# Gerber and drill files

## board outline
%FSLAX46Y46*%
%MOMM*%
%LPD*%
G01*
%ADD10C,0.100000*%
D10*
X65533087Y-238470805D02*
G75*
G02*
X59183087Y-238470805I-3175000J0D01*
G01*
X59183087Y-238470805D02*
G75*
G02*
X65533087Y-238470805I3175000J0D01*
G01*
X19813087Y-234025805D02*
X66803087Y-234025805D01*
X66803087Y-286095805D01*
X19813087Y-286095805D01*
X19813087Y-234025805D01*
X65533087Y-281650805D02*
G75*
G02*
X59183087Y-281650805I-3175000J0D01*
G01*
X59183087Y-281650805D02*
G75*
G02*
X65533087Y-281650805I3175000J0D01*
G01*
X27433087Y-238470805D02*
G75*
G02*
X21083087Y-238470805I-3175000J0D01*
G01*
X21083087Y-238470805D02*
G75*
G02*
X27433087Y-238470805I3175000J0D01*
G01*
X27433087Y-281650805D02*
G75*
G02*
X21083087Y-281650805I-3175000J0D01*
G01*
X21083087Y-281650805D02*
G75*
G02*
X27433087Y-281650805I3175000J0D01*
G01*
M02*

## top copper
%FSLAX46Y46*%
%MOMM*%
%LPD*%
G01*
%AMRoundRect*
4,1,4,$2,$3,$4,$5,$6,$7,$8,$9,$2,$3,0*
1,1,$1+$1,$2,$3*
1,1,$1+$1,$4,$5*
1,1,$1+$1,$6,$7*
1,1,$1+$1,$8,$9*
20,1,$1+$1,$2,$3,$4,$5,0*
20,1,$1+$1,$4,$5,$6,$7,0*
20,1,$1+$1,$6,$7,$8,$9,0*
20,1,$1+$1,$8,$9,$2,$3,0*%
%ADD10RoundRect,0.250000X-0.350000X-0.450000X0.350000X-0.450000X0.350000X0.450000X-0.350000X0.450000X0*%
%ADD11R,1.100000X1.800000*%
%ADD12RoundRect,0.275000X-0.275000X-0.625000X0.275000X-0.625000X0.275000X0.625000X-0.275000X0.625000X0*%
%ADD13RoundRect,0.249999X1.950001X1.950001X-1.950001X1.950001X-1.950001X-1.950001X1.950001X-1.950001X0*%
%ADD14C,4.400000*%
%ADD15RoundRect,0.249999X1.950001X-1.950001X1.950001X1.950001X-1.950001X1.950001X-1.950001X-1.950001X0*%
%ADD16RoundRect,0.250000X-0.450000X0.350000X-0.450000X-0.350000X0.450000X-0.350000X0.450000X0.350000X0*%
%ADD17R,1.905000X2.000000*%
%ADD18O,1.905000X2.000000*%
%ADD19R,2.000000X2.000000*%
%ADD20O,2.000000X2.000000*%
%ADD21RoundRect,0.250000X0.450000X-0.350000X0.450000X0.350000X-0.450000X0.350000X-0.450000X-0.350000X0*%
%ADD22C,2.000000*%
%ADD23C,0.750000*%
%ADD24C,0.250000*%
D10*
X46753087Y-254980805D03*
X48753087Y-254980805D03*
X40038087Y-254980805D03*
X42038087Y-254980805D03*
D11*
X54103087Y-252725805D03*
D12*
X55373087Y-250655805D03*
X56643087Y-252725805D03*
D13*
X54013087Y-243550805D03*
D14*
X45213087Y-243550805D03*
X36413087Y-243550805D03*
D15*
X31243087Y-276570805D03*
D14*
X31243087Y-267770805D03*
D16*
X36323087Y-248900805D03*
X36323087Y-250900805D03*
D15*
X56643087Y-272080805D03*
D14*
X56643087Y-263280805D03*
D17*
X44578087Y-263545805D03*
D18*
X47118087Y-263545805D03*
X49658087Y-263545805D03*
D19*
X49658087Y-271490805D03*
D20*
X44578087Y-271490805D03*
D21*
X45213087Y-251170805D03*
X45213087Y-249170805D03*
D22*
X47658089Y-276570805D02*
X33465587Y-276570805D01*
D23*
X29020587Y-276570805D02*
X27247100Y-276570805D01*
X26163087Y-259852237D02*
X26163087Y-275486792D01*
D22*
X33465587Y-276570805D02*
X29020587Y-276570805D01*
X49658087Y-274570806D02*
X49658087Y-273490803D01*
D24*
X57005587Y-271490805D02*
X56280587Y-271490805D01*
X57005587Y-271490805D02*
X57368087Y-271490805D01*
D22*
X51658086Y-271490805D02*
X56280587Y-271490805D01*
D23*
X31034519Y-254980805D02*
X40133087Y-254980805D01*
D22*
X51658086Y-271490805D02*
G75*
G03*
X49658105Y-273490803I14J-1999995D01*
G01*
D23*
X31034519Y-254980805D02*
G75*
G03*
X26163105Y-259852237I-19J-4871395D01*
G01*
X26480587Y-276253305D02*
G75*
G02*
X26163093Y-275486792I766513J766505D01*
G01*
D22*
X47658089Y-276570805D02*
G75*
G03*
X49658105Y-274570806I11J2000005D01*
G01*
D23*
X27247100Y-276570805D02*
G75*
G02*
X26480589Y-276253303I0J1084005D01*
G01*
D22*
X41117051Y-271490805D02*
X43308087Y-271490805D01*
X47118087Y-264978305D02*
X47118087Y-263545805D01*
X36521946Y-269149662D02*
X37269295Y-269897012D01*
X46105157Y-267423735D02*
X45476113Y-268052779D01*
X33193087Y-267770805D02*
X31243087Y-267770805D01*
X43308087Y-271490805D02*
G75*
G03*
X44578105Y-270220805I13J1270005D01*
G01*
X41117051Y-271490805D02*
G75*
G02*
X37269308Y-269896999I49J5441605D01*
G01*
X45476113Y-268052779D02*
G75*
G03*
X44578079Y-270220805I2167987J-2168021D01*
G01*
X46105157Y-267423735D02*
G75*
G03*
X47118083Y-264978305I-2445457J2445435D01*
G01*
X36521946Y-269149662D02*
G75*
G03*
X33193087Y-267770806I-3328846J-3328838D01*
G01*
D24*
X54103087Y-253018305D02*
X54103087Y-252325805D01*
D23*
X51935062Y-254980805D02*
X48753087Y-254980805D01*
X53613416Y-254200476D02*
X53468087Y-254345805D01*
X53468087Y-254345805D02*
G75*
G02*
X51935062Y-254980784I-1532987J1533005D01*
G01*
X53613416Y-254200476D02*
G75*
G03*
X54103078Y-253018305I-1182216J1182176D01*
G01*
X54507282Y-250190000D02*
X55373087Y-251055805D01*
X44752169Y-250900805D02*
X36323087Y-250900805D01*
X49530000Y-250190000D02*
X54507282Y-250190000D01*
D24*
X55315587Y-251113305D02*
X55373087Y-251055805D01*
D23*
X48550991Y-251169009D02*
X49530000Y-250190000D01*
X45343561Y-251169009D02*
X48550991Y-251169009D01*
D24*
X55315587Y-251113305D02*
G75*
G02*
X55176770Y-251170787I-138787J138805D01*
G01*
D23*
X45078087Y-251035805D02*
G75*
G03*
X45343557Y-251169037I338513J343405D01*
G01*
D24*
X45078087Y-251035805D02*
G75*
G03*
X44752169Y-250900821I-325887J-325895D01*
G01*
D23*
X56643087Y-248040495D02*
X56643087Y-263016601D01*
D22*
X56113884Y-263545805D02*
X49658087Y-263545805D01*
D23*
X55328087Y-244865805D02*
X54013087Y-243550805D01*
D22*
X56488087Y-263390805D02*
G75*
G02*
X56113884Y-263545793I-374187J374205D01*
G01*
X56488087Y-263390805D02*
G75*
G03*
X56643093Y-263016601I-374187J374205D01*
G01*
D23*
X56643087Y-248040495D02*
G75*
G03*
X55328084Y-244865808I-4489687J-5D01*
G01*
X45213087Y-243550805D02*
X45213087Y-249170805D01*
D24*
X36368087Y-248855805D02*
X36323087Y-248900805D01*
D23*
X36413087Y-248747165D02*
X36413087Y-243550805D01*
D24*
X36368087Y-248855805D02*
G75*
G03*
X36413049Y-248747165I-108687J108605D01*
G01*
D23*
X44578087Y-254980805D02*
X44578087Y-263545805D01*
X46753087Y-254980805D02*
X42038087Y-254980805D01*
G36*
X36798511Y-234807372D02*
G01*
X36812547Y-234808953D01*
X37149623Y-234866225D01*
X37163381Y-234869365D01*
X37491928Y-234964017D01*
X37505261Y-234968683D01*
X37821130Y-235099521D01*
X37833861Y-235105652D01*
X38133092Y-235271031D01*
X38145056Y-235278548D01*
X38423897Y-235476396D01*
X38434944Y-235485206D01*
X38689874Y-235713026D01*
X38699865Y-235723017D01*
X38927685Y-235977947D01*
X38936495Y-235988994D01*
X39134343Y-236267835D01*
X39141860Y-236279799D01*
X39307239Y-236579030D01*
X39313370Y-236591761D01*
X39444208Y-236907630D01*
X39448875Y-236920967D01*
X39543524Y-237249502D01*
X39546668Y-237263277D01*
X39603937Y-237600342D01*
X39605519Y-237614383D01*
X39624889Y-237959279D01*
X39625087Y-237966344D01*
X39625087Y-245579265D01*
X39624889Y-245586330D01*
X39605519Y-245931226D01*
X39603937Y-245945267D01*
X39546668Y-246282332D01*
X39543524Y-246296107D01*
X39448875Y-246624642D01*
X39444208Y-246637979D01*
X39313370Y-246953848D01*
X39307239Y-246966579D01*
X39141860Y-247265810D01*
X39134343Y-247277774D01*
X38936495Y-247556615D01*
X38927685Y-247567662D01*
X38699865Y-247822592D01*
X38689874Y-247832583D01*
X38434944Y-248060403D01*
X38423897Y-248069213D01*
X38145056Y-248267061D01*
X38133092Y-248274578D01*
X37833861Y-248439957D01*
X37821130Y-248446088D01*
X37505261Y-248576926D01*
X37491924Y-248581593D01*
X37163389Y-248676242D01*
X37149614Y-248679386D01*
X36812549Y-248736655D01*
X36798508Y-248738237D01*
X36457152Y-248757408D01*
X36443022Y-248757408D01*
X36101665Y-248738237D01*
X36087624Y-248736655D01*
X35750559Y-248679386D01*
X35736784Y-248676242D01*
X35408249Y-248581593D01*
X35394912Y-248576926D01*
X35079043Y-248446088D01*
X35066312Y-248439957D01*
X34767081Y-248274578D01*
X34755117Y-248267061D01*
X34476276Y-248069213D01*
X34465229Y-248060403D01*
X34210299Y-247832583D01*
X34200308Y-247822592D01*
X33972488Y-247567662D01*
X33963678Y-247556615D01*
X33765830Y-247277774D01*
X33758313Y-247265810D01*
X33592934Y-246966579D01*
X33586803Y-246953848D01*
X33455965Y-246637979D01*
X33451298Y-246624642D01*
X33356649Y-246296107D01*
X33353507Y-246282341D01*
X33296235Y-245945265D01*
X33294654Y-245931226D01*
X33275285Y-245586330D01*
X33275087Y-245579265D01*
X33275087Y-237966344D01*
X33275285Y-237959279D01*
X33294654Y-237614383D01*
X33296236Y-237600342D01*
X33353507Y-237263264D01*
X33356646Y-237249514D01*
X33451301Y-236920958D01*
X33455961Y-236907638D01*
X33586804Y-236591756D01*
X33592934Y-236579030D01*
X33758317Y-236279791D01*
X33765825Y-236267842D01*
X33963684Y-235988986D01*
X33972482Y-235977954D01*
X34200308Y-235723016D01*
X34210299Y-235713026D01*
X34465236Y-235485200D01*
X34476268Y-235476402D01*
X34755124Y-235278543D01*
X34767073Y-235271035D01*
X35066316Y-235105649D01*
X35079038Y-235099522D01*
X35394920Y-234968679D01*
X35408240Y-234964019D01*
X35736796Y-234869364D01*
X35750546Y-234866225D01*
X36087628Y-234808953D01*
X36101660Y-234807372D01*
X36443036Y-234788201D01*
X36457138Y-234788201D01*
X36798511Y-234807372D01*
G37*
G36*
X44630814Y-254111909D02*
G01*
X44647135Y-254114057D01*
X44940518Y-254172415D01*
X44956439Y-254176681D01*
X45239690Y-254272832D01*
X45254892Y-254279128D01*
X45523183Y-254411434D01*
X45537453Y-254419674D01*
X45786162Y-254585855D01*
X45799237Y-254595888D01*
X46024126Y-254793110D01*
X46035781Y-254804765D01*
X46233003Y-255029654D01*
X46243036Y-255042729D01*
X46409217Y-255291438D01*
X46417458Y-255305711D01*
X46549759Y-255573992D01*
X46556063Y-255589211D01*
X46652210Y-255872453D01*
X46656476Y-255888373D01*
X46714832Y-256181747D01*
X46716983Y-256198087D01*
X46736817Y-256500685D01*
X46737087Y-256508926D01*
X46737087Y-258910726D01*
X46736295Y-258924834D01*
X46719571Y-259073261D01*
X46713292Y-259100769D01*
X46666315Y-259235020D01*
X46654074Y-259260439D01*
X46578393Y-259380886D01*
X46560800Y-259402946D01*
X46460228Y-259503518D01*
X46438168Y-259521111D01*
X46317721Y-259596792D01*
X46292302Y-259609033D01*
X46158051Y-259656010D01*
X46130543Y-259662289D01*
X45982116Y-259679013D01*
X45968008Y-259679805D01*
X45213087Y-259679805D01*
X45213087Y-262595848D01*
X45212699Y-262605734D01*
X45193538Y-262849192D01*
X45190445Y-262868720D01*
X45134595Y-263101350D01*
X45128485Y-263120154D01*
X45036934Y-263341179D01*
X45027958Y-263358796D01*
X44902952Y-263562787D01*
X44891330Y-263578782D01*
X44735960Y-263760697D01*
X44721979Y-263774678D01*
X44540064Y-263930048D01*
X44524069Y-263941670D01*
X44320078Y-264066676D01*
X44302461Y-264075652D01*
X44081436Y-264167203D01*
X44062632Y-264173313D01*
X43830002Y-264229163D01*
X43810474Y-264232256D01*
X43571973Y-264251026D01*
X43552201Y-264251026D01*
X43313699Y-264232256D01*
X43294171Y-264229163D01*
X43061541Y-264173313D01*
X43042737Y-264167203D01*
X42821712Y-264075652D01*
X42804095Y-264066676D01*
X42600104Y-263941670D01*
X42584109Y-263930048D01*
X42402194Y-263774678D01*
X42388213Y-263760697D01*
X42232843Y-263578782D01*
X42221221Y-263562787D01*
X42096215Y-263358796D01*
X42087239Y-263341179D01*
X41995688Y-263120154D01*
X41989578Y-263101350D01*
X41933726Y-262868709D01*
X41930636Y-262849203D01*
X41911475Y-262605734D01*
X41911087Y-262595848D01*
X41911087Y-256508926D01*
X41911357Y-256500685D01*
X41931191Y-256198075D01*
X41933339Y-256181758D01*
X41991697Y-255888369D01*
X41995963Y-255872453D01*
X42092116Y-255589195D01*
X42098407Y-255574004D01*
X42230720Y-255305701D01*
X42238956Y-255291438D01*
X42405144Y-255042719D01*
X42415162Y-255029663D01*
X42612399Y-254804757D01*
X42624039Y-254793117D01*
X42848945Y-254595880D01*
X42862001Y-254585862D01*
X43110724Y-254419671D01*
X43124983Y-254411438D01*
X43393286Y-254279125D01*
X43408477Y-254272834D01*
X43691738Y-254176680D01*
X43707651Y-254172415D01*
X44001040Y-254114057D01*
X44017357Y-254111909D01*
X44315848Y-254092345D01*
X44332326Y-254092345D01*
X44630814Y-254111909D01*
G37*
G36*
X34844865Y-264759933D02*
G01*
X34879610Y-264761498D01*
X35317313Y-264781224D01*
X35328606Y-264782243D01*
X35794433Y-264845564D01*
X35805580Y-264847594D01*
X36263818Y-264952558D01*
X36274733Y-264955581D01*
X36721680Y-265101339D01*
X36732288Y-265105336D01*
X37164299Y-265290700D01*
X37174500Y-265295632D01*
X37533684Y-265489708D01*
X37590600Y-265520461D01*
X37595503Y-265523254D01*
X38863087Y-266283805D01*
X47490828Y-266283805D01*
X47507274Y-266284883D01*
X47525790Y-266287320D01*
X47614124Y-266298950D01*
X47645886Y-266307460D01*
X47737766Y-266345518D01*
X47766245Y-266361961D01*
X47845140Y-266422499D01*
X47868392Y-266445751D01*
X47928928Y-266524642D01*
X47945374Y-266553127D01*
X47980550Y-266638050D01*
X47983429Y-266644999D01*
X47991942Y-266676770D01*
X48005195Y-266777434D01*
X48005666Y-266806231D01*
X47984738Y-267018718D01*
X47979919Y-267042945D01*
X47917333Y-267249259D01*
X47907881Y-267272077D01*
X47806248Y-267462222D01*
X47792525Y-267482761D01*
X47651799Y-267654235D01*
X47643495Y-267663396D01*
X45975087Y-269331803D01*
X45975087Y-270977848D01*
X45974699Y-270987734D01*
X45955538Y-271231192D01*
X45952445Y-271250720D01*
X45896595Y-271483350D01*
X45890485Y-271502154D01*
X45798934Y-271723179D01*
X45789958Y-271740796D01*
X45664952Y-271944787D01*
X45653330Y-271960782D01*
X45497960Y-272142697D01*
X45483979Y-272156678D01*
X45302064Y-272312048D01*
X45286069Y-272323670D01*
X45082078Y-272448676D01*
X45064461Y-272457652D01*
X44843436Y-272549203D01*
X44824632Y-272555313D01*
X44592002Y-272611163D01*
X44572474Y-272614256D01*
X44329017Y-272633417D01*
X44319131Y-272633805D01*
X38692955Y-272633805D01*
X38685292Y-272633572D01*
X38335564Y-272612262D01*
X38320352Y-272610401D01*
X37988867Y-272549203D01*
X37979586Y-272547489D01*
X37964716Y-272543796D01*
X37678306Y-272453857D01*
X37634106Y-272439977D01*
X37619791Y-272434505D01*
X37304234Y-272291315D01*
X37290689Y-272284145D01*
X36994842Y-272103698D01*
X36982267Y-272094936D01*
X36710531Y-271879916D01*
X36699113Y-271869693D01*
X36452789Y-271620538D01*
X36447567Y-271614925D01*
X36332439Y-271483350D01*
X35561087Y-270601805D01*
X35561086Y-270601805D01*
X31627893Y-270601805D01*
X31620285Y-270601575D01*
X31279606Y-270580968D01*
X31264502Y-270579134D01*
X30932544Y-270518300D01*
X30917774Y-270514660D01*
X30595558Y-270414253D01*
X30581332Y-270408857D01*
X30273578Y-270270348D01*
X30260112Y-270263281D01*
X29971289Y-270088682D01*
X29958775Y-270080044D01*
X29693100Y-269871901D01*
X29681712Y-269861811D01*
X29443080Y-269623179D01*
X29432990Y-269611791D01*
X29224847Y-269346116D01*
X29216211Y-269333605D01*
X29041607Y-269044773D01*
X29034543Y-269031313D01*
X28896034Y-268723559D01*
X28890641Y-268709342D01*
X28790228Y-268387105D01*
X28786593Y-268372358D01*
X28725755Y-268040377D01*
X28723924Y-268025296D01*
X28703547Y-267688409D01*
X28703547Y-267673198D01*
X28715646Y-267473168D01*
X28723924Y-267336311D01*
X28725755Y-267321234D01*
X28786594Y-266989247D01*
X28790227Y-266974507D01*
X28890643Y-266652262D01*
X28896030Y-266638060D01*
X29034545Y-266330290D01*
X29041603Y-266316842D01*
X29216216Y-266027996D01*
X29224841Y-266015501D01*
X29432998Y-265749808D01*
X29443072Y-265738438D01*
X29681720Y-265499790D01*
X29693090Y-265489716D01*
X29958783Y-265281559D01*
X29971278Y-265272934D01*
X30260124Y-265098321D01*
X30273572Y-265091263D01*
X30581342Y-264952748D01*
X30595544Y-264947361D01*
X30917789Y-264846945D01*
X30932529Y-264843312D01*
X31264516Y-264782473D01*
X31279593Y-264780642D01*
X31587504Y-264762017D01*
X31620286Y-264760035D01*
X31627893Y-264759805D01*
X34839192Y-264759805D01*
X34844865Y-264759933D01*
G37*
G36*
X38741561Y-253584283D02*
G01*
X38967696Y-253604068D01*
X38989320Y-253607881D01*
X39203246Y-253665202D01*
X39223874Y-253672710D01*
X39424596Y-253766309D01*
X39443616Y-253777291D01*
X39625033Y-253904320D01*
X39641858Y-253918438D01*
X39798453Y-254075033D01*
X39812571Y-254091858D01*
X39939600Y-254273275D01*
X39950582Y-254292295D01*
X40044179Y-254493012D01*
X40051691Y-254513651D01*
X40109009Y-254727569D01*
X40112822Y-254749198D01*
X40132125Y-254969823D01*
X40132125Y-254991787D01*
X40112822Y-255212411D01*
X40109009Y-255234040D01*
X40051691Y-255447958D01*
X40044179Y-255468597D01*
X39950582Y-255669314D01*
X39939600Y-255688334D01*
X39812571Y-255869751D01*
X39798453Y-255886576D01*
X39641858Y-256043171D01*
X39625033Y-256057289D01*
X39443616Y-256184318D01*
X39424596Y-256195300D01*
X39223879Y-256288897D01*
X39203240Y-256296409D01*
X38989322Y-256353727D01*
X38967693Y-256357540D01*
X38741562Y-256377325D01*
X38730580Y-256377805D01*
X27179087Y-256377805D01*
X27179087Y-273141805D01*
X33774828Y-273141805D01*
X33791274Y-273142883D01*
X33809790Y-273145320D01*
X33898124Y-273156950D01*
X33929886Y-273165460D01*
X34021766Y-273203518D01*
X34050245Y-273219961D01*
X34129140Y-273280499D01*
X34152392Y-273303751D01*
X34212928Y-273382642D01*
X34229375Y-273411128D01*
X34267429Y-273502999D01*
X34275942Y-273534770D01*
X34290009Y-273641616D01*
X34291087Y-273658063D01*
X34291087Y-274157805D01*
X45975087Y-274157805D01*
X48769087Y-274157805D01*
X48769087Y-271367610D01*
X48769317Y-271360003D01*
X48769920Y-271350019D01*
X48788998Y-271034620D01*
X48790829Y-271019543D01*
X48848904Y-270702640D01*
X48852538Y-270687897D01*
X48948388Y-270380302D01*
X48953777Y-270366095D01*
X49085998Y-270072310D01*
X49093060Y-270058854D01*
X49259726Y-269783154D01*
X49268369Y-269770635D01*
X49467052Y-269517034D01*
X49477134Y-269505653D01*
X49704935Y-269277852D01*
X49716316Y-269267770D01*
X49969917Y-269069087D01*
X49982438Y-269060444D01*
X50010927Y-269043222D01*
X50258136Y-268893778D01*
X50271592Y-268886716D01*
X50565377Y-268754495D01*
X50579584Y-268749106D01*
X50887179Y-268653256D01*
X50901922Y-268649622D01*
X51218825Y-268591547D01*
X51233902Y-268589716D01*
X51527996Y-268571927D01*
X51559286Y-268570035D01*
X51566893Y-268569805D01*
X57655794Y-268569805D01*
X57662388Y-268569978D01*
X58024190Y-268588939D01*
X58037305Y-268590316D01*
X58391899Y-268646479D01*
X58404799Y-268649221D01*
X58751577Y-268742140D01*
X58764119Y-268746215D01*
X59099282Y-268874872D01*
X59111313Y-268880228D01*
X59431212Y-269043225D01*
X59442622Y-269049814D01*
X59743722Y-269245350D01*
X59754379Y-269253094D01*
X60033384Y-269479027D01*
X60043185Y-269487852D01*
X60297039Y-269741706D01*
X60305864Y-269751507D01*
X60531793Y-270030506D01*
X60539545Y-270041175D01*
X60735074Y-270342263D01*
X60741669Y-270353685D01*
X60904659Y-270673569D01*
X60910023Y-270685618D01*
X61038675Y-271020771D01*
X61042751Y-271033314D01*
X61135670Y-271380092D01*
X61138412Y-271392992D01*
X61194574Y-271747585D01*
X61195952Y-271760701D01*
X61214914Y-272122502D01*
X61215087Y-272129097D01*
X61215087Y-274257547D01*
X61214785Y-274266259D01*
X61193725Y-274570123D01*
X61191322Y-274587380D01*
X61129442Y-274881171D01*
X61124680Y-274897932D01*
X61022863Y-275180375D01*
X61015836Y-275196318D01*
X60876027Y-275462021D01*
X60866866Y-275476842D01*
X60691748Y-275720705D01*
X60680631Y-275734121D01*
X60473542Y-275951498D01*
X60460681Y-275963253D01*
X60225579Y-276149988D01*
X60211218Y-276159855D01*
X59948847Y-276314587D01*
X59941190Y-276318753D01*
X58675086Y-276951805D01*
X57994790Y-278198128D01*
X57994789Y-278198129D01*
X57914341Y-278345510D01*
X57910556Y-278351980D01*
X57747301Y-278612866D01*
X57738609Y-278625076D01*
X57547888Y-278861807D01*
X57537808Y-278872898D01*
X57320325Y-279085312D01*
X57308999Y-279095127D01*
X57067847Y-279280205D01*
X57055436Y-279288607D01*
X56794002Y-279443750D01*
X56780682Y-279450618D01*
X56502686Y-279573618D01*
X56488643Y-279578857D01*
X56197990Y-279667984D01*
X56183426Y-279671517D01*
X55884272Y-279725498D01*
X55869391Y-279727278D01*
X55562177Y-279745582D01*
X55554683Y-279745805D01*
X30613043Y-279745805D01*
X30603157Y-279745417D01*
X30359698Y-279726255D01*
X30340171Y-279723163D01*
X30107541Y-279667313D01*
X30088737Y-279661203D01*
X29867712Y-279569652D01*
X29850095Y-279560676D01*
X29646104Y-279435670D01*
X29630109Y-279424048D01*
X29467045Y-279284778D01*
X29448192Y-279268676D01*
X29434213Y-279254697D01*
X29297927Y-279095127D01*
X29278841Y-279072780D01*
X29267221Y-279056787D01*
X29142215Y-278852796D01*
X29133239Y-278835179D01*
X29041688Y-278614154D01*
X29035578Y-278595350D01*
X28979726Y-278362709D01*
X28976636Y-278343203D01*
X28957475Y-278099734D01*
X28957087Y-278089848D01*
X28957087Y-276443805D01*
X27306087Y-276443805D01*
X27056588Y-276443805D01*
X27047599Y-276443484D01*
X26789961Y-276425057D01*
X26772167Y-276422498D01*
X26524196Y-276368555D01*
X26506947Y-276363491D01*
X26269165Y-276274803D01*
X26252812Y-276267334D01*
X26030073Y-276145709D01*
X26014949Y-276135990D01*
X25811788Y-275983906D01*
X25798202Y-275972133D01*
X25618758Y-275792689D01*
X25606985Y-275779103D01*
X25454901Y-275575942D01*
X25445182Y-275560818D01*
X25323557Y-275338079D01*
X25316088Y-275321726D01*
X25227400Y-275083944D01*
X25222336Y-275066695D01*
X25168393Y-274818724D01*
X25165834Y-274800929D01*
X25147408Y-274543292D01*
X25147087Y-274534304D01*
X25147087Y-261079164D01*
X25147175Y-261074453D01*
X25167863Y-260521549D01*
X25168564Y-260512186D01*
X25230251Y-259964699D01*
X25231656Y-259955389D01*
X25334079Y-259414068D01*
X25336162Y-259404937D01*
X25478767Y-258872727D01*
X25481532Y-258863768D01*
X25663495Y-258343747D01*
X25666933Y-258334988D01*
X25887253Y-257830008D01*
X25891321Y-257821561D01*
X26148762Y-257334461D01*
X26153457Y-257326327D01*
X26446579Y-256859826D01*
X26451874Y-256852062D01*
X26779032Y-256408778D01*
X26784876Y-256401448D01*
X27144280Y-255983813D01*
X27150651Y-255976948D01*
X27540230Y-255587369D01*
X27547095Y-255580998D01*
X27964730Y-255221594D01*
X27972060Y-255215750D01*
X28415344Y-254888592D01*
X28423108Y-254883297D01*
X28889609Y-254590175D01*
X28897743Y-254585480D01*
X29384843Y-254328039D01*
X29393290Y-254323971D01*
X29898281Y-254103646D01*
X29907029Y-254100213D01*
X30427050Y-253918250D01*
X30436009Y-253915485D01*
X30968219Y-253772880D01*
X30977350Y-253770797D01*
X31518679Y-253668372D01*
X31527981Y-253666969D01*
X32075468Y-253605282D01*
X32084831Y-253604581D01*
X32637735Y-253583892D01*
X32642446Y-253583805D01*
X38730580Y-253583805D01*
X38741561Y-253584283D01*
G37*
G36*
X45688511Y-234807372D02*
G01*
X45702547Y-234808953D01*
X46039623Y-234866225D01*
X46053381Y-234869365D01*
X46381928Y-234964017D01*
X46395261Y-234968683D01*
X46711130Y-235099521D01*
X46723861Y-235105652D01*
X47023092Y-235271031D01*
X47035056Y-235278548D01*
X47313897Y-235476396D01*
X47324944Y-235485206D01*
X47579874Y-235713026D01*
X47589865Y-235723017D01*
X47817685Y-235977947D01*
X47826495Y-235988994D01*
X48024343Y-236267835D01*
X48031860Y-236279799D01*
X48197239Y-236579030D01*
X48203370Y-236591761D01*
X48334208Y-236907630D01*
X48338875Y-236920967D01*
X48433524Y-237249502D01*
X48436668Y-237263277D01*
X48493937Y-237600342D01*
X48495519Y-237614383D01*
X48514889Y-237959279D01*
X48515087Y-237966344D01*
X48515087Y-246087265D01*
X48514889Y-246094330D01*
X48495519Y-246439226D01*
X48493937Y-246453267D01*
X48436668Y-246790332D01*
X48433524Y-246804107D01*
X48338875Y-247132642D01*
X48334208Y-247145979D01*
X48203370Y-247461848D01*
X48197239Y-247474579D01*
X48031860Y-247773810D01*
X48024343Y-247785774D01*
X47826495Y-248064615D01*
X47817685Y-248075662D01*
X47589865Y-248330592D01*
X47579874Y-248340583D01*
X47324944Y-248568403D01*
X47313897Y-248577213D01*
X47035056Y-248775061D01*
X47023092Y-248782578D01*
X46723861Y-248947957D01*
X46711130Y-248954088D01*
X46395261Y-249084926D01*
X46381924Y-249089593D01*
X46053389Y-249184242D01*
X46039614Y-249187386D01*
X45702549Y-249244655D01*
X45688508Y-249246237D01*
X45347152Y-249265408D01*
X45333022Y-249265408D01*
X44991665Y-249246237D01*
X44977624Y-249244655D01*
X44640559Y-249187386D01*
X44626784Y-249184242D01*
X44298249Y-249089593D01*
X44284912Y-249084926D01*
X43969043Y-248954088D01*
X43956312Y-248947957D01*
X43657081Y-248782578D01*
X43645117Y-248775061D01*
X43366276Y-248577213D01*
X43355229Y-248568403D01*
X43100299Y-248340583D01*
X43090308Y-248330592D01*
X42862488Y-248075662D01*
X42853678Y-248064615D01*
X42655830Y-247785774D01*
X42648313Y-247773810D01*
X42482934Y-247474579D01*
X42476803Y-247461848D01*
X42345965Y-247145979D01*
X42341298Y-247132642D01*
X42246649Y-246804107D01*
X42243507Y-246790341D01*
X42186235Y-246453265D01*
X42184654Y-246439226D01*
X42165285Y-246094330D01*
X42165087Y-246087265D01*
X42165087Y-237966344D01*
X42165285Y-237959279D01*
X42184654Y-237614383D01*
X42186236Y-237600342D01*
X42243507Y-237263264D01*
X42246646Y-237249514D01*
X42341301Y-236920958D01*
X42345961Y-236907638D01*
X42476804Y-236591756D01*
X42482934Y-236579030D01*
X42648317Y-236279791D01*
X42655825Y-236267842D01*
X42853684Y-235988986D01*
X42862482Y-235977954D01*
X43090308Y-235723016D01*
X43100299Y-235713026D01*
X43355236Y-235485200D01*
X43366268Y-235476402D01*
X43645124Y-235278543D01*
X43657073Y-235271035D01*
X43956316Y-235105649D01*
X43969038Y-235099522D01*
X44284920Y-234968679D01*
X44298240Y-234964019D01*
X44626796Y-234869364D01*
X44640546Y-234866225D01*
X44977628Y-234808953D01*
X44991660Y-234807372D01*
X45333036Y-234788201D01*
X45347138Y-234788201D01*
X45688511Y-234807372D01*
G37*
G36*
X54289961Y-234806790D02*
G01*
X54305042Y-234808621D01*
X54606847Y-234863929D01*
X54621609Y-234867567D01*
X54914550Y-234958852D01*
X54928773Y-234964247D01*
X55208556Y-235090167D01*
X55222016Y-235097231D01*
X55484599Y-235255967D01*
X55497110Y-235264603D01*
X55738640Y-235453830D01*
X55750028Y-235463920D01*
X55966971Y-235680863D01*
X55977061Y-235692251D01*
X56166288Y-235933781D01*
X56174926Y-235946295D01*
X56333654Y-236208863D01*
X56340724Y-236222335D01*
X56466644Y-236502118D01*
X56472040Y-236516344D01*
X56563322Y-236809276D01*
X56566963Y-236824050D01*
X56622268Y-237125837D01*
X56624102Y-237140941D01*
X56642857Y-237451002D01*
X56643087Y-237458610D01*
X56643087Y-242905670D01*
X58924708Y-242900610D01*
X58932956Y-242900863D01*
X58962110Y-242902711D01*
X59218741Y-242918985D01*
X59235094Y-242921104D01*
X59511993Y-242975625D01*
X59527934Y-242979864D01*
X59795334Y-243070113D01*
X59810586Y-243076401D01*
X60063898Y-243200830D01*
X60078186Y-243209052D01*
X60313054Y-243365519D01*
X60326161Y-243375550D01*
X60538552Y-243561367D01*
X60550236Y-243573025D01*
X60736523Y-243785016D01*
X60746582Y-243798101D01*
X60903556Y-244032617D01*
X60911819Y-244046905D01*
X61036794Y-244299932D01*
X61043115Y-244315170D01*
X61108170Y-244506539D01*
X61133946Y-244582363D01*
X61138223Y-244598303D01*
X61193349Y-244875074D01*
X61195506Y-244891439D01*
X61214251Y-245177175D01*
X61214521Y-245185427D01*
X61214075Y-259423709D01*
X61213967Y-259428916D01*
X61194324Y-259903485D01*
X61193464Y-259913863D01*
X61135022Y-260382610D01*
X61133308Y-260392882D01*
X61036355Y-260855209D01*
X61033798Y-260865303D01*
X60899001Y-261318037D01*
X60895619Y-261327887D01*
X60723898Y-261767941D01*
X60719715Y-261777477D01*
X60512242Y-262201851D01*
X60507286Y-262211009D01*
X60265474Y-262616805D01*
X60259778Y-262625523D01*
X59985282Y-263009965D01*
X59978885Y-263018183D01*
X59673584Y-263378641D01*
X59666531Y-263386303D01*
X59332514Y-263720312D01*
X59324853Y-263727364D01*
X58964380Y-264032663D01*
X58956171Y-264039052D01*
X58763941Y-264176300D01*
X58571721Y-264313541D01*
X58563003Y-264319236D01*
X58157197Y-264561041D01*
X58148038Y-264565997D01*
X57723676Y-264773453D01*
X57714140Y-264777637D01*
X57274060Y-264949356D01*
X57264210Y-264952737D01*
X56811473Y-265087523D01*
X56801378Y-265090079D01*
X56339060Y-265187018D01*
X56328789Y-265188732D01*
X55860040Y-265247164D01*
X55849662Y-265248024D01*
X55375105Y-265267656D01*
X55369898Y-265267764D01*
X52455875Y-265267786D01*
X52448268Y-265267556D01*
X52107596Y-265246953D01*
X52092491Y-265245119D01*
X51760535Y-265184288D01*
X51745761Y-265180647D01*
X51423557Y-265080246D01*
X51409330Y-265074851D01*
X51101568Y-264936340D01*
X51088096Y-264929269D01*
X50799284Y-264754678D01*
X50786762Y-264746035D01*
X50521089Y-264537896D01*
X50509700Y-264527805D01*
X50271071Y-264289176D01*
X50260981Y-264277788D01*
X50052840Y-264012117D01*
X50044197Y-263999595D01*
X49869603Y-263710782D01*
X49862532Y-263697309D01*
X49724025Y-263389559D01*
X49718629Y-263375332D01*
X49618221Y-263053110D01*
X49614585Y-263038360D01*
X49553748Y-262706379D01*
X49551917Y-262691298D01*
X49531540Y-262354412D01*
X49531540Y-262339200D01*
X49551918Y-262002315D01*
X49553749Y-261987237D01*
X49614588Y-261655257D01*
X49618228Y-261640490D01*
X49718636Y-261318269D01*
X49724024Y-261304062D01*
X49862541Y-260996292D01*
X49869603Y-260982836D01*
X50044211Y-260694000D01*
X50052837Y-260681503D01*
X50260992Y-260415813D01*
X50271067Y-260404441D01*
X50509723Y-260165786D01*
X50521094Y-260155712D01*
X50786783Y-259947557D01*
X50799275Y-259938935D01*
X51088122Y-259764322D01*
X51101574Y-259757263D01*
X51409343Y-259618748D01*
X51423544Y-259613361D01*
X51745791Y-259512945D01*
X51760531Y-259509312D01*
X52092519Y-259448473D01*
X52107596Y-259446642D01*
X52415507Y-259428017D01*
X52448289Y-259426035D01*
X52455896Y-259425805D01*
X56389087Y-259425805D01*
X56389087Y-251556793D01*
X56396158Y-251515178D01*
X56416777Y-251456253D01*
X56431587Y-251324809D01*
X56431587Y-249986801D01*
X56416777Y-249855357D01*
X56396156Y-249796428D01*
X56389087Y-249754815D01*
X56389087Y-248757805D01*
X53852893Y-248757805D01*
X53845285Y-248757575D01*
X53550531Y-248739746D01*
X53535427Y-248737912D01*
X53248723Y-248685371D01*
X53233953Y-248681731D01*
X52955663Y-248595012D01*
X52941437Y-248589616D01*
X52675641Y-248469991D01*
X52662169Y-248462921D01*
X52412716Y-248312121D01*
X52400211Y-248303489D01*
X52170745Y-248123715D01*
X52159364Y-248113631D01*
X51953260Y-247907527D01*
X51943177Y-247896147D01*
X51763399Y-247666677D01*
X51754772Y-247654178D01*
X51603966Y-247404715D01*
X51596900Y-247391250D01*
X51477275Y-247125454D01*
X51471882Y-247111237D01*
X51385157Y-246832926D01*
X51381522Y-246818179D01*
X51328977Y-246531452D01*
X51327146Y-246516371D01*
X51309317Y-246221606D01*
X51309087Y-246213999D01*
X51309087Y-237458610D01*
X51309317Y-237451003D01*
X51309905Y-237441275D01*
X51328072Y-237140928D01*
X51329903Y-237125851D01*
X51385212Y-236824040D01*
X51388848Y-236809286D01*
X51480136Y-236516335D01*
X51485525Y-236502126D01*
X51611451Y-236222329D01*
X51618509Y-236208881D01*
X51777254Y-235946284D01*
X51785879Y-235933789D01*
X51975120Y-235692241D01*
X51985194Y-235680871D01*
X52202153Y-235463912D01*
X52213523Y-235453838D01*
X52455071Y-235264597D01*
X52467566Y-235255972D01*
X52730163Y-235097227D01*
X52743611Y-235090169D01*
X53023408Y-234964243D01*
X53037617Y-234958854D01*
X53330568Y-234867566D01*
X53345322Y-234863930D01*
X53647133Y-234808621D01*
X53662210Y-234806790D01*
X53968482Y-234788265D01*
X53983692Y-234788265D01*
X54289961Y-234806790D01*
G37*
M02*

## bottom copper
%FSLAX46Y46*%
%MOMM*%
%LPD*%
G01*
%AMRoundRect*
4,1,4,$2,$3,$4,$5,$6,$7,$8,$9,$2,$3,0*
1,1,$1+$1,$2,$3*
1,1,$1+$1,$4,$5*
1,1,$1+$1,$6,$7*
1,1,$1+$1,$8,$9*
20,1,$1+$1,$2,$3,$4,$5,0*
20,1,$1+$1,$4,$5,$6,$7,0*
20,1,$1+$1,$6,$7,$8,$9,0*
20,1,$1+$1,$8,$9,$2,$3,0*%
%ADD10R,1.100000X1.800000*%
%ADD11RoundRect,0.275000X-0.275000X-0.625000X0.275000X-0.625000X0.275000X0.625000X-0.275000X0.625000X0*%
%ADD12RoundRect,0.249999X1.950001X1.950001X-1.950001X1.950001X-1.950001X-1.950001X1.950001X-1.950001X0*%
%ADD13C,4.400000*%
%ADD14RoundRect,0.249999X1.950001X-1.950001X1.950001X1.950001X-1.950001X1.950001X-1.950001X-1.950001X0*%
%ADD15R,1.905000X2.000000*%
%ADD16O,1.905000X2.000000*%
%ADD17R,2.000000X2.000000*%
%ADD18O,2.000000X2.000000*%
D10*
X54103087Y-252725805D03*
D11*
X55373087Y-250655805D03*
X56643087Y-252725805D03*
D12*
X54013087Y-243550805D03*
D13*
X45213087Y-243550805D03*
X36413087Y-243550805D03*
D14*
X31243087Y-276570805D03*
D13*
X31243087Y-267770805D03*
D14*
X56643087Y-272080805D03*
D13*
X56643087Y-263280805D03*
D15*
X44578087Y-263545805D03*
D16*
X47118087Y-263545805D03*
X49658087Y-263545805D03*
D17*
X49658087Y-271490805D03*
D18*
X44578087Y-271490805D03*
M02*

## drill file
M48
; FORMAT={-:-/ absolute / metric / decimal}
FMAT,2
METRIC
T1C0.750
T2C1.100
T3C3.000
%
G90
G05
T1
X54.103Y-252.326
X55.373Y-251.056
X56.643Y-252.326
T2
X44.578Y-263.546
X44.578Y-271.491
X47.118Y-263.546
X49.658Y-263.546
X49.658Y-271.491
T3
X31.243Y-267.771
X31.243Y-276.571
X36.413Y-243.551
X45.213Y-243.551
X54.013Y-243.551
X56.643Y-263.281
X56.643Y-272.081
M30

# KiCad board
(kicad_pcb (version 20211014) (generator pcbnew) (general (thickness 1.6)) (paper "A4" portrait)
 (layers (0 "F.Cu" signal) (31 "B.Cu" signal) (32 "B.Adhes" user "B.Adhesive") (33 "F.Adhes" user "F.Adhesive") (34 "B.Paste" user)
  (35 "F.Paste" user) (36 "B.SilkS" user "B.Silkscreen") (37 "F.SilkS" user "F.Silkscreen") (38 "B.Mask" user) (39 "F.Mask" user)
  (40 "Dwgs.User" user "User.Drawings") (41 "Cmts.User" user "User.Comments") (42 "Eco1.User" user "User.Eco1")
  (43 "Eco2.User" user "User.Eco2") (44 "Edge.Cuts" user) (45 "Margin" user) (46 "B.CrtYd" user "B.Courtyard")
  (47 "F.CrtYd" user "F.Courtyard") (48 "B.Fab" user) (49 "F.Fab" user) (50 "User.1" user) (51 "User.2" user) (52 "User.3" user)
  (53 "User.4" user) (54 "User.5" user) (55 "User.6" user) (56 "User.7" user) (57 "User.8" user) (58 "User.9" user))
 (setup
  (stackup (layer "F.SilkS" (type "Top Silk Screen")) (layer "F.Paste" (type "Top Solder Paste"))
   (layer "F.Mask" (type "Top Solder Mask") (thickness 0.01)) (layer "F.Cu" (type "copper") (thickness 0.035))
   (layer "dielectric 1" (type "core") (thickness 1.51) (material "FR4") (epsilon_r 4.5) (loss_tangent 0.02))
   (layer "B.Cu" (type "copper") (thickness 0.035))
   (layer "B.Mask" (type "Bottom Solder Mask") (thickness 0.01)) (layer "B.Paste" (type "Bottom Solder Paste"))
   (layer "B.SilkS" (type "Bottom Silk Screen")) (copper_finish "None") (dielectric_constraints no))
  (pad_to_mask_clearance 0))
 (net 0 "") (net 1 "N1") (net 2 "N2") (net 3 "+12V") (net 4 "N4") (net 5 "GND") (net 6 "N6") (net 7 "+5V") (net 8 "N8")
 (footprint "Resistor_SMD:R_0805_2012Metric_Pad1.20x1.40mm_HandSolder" (layer "F.Cu") (at 47.753087 254.980805)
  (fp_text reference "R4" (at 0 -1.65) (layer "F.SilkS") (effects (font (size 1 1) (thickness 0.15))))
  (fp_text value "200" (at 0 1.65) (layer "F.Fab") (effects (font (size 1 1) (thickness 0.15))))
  (pad "1" smd roundrect (at -1 0) (size 1.2 1.4) (layers "F.Cu" "F.Paste" "F.Mask") (roundrect_rratio 0.2083333333) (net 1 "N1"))
  (pad "2" smd roundrect (at 1 0) (size 1.2 1.4) (layers "F.Cu" "F.Paste" "F.Mask") (roundrect_rratio 0.2083333333) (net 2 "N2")))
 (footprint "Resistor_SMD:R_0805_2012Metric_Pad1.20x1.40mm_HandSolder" (layer "F.Cu") (at 41.038087 254.980805)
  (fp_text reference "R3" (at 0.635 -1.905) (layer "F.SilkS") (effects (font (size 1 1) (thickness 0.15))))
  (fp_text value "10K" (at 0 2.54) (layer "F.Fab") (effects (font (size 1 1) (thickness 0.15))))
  (pad "1" smd roundrect (at -1 0) (size 1.2 1.4) (layers "F.Cu" "F.Paste" "F.Mask") (roundrect_rratio 0.2083333333) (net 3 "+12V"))
  (pad "2" smd roundrect (at 1 0) (size 1.2 1.4) (layers "F.Cu" "F.Paste" "F.Mask") (roundrect_rratio 0.2083333333) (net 1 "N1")))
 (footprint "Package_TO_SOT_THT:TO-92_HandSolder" (layer "F.Cu") (at 54.103087 252.325805)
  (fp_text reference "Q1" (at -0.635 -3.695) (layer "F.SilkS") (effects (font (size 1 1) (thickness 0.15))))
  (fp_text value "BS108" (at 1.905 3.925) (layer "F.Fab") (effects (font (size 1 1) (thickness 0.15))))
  (pad "1" thru_hole rect (at 0 0) (size 1.1 1.8) (drill 0.75 (offset 0 0.4)) (layers *.Cu *.Mask) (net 2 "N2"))
  (pad "2" thru_hole roundrect (at 1.27 -1.27) (size 1.1 1.8) (drill 0.75 (offset 0 -0.4)) (layers *.Cu *.Mask) (roundrect_rratio 0.25)
   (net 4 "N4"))
  (pad "3" thru_hole roundrect (at 2.54 0) (size 1.1 1.8) (drill 0.75 (offset 0 0.4)) (layers *.Cu *.Mask) (roundrect_rratio 0.25)
   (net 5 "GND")))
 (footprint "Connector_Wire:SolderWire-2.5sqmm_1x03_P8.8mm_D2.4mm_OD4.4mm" (layer "F.Cu") (at 54.013087 243.550805 180)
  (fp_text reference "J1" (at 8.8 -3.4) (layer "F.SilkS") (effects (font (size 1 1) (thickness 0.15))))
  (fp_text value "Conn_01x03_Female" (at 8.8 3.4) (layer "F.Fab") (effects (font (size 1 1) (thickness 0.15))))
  (pad "1" thru_hole roundrect (at 0 0 180) (size 4.4 4.4) (drill 3) (layers *.Cu *.Mask) (roundrect_rratio 0.05681795455) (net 5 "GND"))
  (pad "2" thru_hole circle (at 8.8 0 180) (size 4.4 4.4) (drill 3) (layers *.Cu *.Mask) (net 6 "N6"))
  (pad "3" thru_hole circle (at 17.6 0 180) (size 4.4 4.4) (drill 3) (layers *.Cu *.Mask) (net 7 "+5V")))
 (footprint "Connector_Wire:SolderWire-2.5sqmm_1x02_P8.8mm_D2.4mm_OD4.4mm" (layer "F.Cu") (at 31.243087 276.570805 90)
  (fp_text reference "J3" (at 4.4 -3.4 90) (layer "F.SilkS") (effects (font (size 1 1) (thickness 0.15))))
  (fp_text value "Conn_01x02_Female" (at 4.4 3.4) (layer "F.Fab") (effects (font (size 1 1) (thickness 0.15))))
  (pad "1" thru_hole roundrect (at 0 0 90) (size 4.4 4.4) (drill 3) (layers *.Cu *.Mask) (roundrect_rratio 0.05681795455) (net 3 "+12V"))
  (pad "2" thru_hole circle (at 8.8 0 90) (size 4.4 4.4) (drill 3) (layers *.Cu *.Mask) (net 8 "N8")))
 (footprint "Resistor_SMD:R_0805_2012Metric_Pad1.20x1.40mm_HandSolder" (layer "F.Cu") (at 36.323087 249.900805 -90)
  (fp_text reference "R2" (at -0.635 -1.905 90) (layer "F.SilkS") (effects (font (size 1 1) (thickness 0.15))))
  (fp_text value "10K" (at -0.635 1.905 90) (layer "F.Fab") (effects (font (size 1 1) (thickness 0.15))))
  (pad "1" smd roundrect (at -1 0 270) (size 1.2 1.4) (layers "F.Cu" "F.Paste" "F.Mask") (roundrect_rratio 0.2083333333) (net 7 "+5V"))
  (pad "2" smd roundrect (at 1 0 270) (size 1.2 1.4) (layers "F.Cu" "F.Paste" "F.Mask") (roundrect_rratio 0.2083333333) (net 4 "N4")))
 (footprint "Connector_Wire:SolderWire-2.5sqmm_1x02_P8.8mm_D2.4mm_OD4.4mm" (layer "F.Cu") (at 56.643087 272.080805 90)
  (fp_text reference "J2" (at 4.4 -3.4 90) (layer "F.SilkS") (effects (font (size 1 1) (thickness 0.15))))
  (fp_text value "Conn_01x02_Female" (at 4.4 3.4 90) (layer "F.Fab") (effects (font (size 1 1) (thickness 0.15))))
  (pad "1" thru_hole roundrect (at 0 0 90) (size 4.4 4.4) (drill 3) (layers *.Cu *.Mask) (roundrect_rratio 0.05681795455) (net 3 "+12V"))
  (pad "2" thru_hole circle (at 8.8 0 90) (size 4.4 4.4) (drill 3) (layers *.Cu *.Mask) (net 5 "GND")))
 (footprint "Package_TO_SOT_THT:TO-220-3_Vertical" (layer "F.Cu") (at 44.578087 263.545805)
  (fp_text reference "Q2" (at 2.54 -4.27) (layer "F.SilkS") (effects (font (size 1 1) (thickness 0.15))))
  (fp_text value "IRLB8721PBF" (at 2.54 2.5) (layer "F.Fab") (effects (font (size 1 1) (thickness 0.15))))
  (pad "1" thru_hole rect (at 0 0) (size 1.905 2) (drill 1.1) (layers *.Cu *.Mask) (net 1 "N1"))
  (pad "2" thru_hole oval (at 2.54 0) (size 1.905 2) (drill 1.1) (layers *.Cu *.Mask) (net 8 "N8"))
  (pad "3" thru_hole oval (at 5.08 0) (size 1.905 2) (drill 1.1) (layers *.Cu *.Mask) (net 5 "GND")))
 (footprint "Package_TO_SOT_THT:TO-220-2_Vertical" (layer "F.Cu") (at 49.658087 271.490805 180)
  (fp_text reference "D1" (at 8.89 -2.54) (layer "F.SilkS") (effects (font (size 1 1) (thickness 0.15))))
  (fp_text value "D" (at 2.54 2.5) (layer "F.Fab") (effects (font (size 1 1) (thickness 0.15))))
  (pad "1" thru_hole rect (at 0 0 180) (size 2 2) (drill 1.1) (layers *.Cu *.Mask) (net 3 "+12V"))
  (pad "2" thru_hole oval (at 5.08 0 180) (size 2 2) (drill 1.1) (layers *.Cu *.Mask) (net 8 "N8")))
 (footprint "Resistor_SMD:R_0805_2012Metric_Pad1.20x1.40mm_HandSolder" (layer "F.Cu") (at 45.213087 250.170805 90)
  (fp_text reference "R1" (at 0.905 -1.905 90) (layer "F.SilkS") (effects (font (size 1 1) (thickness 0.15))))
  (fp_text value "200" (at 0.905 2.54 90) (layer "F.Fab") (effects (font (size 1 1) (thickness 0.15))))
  (pad "1" smd roundrect (at -1 0 90) (size 1.2 1.4) (layers "F.Cu" "F.Paste" "F.Mask") (roundrect_rratio 0.2083333333) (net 4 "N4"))
  (pad "2" smd roundrect (at 1 0 90) (size 1.2 1.4) (layers "F.Cu" "F.Paste" "F.Mask") (roundrect_rratio 0.2083333333) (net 6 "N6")))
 (gr_circle (center 62.358087 238.470805) (end 64.898087 240.375805) (layer "Edge.Cuts") (width 0.1) (fill none))
 (gr_rect (start 19.813087 234.025805) (end 66.803087 286.095805) (layer "Edge.Cuts") (width 0.1) (fill none))
 (gr_circle (center 62.358087 281.650805) (end 64.898087 283.555805) (layer "Edge.Cuts") (width 0.1) (fill none))
 (gr_circle (center 24.258087 238.470805) (end 26.798087 240.375805) (layer "Edge.Cuts") (width 0.1) (fill none))
 (gr_circle (center 24.258087 281.650805) (end 26.798087 283.555805) (layer "Edge.Cuts") (width 0.1) (fill none))
 (segment (start 47.658089 276.570805) (end 33.465587 276.570805) (width 2) (layer "F.Cu") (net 3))
 (segment (start 29.020587 276.570805) (end 27.2471 276.570805) (width 0.75) (layer "F.Cu") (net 3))
 (segment (start 26.163087 259.852237) (end 26.163087 275.486792) (width 0.75) (layer "F.Cu") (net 3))
 (segment (start 33.465587 276.570805) (end 29.020587 276.570805) (width 2) (layer "F.Cu") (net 3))
 (segment (start 49.658087 274.570806) (end 49.658087 273.490803) (width 2) (layer "F.Cu") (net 3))
 (segment (start 57.005587 271.490805) (end 56.280587 271.490805) (width 0.25) (layer "F.Cu") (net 3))
 (segment (start 57.005587 271.490805) (end 57.368087 271.490805) (width 0.25) (layer "F.Cu") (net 3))
 (segment (start 51.658086 271.490805) (end 56.280587 271.490805) (width 2) (layer "F.Cu") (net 3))
 (segment (start 31.034519 254.980805) (end 40.133087 254.980805) (width 0.75) (layer "F.Cu") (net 3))
 (arc (start 51.658086 271.490805) (mid 50.243874 272.07659) (end 49.658087 273.490803) (width 2) (layer "F.Cu") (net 3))
 (arc (start 31.034519 254.980805) (mid 27.589896 256.407614) (end 26.163087 259.852237) (width 0.75) (layer "F.Cu") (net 3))
 (arc (start 26.480587 276.253305) (mid 26.245603 275.901625) (end 26.163087 275.486792) (width 0.75) (layer "F.Cu") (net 3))
 (arc (start 47.658089 276.570805) (mid 49.072302 275.985018) (end 49.658087 274.570806) (width 2) (layer "F.Cu") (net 3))
 (arc (start 27.2471 276.570805) (mid 26.832267 276.488289) (end 26.480587 276.253305) (width 0.75) (layer "F.Cu") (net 3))
 (segment (start 41.117051 271.490805) (end 43.308087 271.490805) (width 2) (layer "F.Cu") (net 8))
 (segment (start 47.118087 264.978305) (end 47.118087 263.545805) (width 2) (layer "F.Cu") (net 8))
 (segment (start 36.521946 269.149662) (end 37.269295 269.897012) (width 2) (layer "F.Cu") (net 8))
 (segment (start 46.105157 267.423735) (end 45.476113 268.052779) (width 2) (layer "F.Cu") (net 8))
 (segment (start 33.193087 267.770805) (end 31.243087 267.770805) (width 2) (layer "F.Cu") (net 8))
 (arc (start 43.308087 271.490805) (mid 44.206113 271.11883) (end 44.578087 270.220805) (width 2) (layer "F.Cu") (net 8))
 (arc (start 41.117051 271.490805) (mid 39.034661 271.076591) (end 37.269295 269.897012) (width 2) (layer "F.Cu") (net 8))
 (arc (start 45.476113 268.052779) (mid 44.811477 269.047477) (end 44.578087 270.220805) (width 2) (layer "F.Cu") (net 8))
 (arc (start 46.105157 267.423735) (mid 46.854836 266.301762) (end 47.118087 264.978305) (width 2) (layer "F.Cu") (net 8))
 (arc (start 36.521946 269.149662) (mid 34.994653 268.129158) (end 33.193087 267.770805) (width 2) (layer "F.Cu") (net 8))
 (segment (start 54.103087 253.018305) (end 54.103087 252.325805) (width 0.25) (layer "F.Cu") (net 2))
 (segment (start 51.935062 254.980805) (end 48.753087 254.980805) (width 0.75) (layer "F.Cu") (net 2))
 (segment (start 53.613416 254.200476) (end 53.468087 254.345805) (width 0.75) (layer "F.Cu") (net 2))
 (arc (start 53.468087 254.345805) (mid 52.76473 254.815773) (end 51.935062 254.980805) (width 0.75) (layer "F.Cu") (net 2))
 (arc (start 53.613416 254.200476) (mid 53.975826 253.658091) (end 54.103087 253.018305) (width 0.75) (layer "F.Cu") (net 2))
 (segment (start 54.507282 250.19) (end 55.373087 251.055805) (width 0.75) (layer "F.Cu") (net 4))
 (segment (start 44.752169 250.900805) (end 36.323087 250.900805) (width 0.75) (layer "F.Cu") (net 4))
 (segment (start 49.53 250.19) (end 54.507282 250.19) (width 0.75) (layer "F.Cu") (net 4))
 (segment (start 55.315587 251.113305) (end 55.373087 251.055805) (width 0.25) (layer "F.Cu") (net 4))
 (segment (start 48.550991 251.169009) (end 49.53 250.19) (width 0.75) (layer "F.Cu") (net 4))
 (segment (start 45.343561 251.169009) (end 48.550991 251.169009) (width 0.75) (layer "F.Cu") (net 4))
 (arc (start 55.315587 251.113305) (mid 55.251898 251.155861) (end 55.17677 251.170805) (width 0.25) (layer "F.Cu") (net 4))
 (arc (start 45.078087 251.035805) (mid 45.200146 251.123273) (end 45.343561 251.169009) (width 0.75) (layer "F.Cu") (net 4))
 (arc (start 45.078087 251.035805) (mid 44.928555 250.93589) (end 44.752169 250.900805) (width 0.25) (layer "F.Cu") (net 4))
 (segment (start 56.643087 248.040495) (end 56.643087 263.016601) (width 0.75) (layer "F.Cu") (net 5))
 (segment (start 56.113884 263.545805) (end 49.658087 263.545805) (width 2) (layer "F.Cu") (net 5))
 (segment (start 55.328087 244.865805) (end 54.013087 243.550805) (width 0.75) (layer "F.Cu") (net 5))
 (arc (start 56.488087 263.390805) (mid 56.316402 263.505521) (end 56.113884 263.545805) (width 2) (layer "F.Cu") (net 5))
 (arc (start 56.488087 263.390805) (mid 56.602804 263.219118) (end 56.643087 263.016601) (width 2) (layer "F.Cu") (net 5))
 (arc (start 56.643087 248.040495) (mid 56.30133 246.322365) (end 55.328087 244.865805) (width 0.75) (layer "F.Cu") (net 5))
 (segment (start 45.213087 243.550805) (end 45.213087 249.170805) (width 0.75) (layer "F.Cu") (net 6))
 (segment (start 36.368087 248.855805) (end 36.323087 248.900805) (width 0.25) (layer "F.Cu") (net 7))
 (segment (start 36.413087 248.747165) (end 36.413087 243.550805) (width 0.75) (layer "F.Cu") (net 7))
 (arc (start 36.368087 248.855805) (mid 36.401392 248.80596) (end 36.413087 248.747165) (width 0.25) (layer "F.Cu") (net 7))
 (segment (start 44.578087 254.980805) (end 44.578087 263.545805) (width 0.75) (layer "F.Cu") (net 1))
 (segment (start 46.753087 254.980805) (end 42.038087 254.980805) (width 0.75) (layer "F.Cu") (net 1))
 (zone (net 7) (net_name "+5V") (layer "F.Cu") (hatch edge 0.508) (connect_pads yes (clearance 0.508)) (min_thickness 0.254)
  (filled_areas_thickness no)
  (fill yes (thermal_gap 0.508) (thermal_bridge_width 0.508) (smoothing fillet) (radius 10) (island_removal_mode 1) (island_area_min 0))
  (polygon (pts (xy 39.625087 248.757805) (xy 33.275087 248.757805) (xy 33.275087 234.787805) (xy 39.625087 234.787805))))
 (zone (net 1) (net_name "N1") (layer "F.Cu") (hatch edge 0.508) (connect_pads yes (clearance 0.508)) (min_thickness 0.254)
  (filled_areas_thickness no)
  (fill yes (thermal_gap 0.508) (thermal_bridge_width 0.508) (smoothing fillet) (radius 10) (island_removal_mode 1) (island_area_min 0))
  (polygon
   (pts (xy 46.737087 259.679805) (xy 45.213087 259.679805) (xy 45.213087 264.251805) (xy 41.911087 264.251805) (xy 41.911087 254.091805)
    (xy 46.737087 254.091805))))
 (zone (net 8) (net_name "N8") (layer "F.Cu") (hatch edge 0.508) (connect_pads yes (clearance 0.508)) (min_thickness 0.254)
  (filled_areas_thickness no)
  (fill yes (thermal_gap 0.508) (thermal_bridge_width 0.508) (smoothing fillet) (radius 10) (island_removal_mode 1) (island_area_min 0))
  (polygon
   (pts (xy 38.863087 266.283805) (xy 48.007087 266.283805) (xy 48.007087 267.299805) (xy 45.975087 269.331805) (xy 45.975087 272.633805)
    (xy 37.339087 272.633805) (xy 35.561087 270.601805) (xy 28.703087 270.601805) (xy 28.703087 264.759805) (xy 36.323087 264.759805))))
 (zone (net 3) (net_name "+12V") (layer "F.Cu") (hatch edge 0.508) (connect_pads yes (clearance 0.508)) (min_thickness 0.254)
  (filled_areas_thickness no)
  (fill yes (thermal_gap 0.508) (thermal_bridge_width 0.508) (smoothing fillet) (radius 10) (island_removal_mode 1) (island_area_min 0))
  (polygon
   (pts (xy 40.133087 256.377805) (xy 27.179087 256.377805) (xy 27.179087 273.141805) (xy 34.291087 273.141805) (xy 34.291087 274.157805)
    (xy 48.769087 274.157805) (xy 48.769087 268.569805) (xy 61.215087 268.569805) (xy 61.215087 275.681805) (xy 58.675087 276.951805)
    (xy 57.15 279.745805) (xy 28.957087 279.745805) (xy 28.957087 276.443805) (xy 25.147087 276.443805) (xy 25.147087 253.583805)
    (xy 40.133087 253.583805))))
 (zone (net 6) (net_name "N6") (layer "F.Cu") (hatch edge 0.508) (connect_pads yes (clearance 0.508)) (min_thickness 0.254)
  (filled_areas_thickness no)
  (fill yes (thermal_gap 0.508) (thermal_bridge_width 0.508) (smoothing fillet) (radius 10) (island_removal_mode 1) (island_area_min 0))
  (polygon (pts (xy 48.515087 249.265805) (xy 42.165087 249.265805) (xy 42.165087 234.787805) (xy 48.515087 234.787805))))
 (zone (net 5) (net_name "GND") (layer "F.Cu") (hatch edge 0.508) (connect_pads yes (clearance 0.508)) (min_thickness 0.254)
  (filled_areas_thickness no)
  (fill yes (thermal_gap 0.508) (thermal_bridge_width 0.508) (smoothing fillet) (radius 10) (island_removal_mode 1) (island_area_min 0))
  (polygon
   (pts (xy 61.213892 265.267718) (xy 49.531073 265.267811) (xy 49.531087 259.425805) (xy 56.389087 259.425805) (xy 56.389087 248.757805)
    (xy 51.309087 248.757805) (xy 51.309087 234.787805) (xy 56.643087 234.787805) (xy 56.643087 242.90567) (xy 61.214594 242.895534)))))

